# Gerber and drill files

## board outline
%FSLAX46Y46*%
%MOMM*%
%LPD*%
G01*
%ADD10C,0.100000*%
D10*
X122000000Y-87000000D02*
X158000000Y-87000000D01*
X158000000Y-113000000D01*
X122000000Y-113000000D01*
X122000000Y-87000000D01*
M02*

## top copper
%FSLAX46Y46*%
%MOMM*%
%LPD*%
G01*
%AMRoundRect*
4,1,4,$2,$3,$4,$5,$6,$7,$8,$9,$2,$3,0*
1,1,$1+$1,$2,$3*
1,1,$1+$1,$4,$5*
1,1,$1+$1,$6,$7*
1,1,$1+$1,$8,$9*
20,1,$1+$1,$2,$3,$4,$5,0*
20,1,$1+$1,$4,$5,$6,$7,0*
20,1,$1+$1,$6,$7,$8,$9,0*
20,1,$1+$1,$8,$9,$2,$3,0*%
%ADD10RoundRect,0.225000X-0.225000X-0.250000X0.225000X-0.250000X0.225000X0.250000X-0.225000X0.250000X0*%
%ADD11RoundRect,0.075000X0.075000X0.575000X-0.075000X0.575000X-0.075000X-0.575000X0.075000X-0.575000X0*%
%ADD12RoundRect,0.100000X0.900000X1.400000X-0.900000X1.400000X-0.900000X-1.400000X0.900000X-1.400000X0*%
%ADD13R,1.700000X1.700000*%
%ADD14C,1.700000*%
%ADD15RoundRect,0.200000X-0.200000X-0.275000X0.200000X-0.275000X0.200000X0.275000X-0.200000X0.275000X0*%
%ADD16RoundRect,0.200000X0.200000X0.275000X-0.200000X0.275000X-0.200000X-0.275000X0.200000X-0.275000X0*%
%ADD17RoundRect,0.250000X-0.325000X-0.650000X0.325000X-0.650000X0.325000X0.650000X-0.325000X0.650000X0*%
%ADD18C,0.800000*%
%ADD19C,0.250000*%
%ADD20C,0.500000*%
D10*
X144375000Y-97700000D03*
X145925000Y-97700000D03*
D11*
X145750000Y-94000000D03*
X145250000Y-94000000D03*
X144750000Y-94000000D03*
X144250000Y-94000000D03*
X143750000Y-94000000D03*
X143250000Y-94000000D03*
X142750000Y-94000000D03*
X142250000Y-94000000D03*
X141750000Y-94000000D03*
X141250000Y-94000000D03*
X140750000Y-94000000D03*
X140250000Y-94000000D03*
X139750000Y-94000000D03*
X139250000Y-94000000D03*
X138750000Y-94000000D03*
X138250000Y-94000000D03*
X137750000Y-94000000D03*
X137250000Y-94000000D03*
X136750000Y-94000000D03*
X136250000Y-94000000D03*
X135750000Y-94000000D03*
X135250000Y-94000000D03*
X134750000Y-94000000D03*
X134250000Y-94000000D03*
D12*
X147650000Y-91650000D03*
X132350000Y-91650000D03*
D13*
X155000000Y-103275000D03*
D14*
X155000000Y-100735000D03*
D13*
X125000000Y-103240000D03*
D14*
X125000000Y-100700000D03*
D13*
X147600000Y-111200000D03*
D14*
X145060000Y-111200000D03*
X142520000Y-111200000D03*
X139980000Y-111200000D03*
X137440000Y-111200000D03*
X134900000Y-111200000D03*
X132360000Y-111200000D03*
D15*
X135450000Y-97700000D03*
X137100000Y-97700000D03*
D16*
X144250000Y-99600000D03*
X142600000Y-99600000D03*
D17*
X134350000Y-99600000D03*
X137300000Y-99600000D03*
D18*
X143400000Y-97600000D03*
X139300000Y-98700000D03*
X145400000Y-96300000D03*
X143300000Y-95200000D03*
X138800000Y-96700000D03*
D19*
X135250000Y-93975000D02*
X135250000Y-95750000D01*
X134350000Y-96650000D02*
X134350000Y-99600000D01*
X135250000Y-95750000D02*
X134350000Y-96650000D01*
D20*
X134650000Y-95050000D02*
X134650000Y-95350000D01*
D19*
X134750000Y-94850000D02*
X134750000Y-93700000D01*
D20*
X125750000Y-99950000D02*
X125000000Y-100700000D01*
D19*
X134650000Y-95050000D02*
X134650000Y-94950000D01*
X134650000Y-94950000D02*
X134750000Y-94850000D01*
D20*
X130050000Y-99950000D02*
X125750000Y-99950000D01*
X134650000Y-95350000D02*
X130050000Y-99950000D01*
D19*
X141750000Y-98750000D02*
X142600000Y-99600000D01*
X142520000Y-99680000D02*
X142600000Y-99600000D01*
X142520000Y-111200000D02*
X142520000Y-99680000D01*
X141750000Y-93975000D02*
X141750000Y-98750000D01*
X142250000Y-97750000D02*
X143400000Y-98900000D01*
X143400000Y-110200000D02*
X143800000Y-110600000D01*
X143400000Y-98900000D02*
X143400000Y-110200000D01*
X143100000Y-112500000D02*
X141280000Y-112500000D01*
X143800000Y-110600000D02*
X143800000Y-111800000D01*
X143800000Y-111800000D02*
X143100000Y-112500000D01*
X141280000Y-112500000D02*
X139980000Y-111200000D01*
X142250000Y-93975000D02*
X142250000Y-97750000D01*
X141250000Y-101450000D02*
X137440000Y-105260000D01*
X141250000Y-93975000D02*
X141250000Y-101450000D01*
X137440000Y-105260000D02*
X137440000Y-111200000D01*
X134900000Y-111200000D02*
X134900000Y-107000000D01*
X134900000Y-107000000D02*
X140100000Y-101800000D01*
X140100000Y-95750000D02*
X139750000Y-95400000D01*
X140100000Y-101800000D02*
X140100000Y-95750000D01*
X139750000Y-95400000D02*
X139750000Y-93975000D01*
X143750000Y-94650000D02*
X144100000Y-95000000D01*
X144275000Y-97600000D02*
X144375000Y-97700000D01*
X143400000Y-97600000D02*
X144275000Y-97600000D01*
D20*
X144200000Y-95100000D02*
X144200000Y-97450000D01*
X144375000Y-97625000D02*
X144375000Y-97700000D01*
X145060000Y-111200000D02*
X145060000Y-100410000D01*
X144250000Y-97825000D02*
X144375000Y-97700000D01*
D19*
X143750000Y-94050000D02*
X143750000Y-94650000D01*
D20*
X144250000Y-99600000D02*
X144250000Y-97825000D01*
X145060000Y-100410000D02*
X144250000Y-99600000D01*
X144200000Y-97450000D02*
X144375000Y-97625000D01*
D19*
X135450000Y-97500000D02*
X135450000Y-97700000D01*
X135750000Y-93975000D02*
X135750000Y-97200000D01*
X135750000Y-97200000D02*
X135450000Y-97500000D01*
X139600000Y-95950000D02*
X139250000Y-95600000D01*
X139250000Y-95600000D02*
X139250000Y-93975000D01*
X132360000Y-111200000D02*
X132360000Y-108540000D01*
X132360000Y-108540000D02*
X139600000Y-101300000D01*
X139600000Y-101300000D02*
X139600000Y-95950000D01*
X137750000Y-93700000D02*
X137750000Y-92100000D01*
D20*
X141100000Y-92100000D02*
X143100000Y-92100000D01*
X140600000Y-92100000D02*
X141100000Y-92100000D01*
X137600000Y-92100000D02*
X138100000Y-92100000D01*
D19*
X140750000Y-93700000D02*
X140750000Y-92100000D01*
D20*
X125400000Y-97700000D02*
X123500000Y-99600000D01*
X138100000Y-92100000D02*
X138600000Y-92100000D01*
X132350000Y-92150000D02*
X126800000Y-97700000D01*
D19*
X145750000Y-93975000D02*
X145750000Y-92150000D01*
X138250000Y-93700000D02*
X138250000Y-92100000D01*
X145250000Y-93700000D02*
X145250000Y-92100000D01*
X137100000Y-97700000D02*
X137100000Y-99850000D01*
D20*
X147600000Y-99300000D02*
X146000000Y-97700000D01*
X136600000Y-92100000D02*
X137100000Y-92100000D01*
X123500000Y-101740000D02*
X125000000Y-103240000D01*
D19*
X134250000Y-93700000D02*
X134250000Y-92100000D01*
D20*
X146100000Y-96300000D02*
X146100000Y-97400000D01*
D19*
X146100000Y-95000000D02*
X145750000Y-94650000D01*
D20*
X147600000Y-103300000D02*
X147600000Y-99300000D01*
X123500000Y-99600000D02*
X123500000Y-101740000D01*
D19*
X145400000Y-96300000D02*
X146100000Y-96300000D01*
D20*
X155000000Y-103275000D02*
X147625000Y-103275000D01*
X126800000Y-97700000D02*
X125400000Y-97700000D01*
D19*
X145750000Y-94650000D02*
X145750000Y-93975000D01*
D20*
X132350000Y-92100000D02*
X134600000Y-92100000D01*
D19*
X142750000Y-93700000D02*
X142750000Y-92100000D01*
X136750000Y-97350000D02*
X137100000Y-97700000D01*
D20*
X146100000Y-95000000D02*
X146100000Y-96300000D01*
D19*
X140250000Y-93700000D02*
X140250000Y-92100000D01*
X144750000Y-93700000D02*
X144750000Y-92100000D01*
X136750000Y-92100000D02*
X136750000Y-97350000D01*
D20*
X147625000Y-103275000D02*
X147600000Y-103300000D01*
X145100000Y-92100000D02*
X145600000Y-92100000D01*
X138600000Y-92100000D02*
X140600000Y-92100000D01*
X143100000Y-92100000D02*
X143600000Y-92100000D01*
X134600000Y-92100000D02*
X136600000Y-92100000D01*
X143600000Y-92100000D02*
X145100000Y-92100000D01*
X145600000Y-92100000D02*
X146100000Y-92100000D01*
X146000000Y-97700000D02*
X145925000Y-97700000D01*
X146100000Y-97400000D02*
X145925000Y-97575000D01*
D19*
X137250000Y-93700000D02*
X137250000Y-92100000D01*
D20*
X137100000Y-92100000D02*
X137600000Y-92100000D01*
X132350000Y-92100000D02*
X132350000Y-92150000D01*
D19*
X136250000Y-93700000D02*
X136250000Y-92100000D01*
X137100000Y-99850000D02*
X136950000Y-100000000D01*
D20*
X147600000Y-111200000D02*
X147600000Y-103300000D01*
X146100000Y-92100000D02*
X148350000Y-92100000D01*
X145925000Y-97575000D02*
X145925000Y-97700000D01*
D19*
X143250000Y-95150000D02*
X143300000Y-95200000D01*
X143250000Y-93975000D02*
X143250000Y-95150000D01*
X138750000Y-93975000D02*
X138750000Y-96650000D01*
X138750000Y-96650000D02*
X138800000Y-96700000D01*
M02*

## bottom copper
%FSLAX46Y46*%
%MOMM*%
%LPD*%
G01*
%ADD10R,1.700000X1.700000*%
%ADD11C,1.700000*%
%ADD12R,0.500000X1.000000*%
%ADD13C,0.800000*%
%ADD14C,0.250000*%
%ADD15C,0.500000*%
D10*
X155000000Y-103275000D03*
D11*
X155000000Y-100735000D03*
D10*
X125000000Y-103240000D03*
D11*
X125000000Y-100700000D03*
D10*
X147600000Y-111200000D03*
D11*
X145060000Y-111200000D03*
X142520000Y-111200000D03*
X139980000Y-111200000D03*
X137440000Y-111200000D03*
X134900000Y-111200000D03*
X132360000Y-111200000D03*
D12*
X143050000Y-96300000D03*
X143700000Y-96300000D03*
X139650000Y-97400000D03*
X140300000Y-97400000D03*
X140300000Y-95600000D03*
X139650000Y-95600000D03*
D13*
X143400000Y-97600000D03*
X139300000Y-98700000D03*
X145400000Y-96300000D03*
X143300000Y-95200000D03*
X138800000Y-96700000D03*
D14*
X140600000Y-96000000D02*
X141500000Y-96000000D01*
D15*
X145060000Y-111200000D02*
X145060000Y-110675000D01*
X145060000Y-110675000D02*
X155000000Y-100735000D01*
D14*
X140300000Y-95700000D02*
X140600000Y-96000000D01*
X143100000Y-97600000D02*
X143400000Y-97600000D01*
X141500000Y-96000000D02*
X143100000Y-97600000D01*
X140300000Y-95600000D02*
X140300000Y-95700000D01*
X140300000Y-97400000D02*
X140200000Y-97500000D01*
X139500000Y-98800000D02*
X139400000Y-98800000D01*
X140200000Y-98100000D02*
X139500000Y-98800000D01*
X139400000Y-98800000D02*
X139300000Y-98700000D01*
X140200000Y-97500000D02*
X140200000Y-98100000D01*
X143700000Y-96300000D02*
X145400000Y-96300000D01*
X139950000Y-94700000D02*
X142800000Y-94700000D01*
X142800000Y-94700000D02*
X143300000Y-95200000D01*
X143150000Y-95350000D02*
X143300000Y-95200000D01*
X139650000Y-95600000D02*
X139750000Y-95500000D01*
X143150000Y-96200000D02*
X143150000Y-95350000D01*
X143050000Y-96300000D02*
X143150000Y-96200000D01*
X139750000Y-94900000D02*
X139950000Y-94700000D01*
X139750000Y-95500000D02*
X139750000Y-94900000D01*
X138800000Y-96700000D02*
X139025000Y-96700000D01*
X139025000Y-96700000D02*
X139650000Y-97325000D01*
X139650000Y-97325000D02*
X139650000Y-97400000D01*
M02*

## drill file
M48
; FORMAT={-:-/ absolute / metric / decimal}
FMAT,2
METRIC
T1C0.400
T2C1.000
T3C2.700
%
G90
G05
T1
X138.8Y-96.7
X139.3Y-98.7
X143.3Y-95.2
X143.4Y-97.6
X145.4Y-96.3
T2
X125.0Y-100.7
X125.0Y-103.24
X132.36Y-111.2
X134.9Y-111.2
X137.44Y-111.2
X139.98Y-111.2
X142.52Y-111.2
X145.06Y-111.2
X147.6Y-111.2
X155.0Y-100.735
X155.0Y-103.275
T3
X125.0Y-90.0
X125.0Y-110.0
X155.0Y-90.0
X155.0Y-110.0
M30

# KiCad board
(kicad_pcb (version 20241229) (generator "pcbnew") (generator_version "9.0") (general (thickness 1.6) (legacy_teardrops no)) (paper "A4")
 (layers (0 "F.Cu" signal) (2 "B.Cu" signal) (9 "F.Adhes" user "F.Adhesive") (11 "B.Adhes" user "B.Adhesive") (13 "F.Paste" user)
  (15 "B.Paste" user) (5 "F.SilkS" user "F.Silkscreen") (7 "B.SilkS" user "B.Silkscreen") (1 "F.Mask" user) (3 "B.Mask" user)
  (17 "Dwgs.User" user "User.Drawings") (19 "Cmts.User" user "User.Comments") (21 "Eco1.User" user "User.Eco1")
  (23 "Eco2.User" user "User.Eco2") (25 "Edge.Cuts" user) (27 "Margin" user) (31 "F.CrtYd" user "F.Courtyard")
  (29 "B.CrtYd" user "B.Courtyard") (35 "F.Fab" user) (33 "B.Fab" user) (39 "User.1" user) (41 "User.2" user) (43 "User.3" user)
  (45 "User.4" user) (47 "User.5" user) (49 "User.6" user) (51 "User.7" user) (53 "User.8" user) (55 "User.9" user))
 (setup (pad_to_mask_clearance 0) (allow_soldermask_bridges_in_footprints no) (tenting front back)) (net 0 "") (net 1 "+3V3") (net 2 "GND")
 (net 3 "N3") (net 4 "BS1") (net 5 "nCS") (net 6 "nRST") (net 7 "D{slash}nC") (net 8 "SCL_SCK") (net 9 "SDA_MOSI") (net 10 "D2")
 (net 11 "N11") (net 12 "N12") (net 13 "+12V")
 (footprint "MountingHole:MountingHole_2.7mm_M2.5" (layer "F.Cu") (at 155 110)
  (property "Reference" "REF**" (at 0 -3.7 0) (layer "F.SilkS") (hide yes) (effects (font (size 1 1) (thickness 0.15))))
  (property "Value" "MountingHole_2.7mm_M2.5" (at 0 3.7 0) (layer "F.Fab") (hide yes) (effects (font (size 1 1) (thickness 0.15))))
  (pad "" np_thru_hole circle (at 0 0) (size 2.7 2.7) (drill 2.7) (layers "*.Cu" "*.Mask")))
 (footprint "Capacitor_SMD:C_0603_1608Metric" (layer "F.Cu") (at 145.15 97.7)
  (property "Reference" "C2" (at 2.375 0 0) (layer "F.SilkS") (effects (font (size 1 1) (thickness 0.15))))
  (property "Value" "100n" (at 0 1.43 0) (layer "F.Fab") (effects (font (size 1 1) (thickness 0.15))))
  (pad "1" smd roundrect (at -0.775 0) (size 0.9 0.95) (layers "F.Cu" "F.Mask" "F.Paste") (roundrect_rratio 0.25) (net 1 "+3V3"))
  (pad "2" smd roundrect (at 0.775 0) (size 0.9 0.95) (layers "F.Cu" "F.Mask" "F.Paste") (roundrect_rratio 0.25) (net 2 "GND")))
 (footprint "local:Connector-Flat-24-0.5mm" (layer "F.Cu") (at 140 92.9 180)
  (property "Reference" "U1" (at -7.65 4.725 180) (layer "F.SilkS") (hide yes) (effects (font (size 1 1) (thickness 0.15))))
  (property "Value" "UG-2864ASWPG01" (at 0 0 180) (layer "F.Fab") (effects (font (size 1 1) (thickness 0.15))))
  (pad "1" smd roundrect (at -5.75 -1.1 180) (size 0.3 1.3) (layers "F.Cu" "F.Mask" "F.Paste") (roundrect_rratio 0.25) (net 2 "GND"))
  (pad "2" smd roundrect (at -5.25 -1.1 180) (size 0.3 1.3) (layers "F.Cu" "F.Mask" "F.Paste") (roundrect_rratio 0.25) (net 2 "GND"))
  (pad "3" smd roundrect (at -4.75 -1.1 180) (size 0.3 1.3) (layers "F.Cu" "F.Mask" "F.Paste") (roundrect_rratio 0.25) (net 2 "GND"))
  (pad "4" smd roundrect (at -4.25 -1.1 180) (size 0.3 1.3) (layers "F.Cu" "F.Mask" "F.Paste") (roundrect_rratio 0.25) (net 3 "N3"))
  (pad "5" smd roundrect (at -3.75 -1.1 180) (size 0.3 1.3) (layers "F.Cu" "F.Mask" "F.Paste") (roundrect_rratio 0.25) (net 1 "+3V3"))
  (pad "6" smd roundrect (at -3.25 -1.1 180) (size 0.3 1.3) (layers "F.Cu" "F.Mask" "F.Paste") (roundrect_rratio 0.25) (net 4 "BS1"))
  (pad "7" smd roundrect (at -2.75 -1.1 180) (size 0.3 1.3) (layers "F.Cu" "F.Mask" "F.Paste") (roundrect_rratio 0.25) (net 2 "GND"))
  (pad "8" smd roundrect (at -2.25 -1.1 180) (size 0.3 1.3) (layers "F.Cu" "F.Mask" "F.Paste") (roundrect_rratio 0.25) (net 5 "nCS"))
  (pad "9" smd roundrect (at -1.75 -1.1 180) (size 0.3 1.3) (layers "F.Cu" "F.Mask" "F.Paste") (roundrect_rratio 0.25) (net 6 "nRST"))
  (pad "10" smd roundrect (at -1.25 -1.1 180) (size 0.3 1.3) (layers "F.Cu" "F.Mask" "F.Paste") (roundrect_rratio 0.25) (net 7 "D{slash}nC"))
  (pad "11" smd roundrect (at -0.75 -1.1 180) (size 0.3 1.3) (layers "F.Cu" "F.Mask" "F.Paste") (roundrect_rratio 0.25) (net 2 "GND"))
  (pad "12" smd roundrect (at -0.25 -1.1 180) (size 0.3 1.3) (layers "F.Cu" "F.Mask" "F.Paste") (roundrect_rratio 0.25) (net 2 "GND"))
  (pad "13" smd roundrect (at 0.25 -1.1 180) (size 0.3 1.3) (layers "F.Cu" "F.Mask" "F.Paste") (roundrect_rratio 0.25) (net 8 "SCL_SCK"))
  (pad "14" smd roundrect (at 0.75 -1.1 180) (size 0.3 1.3) (layers "F.Cu" "F.Mask" "F.Paste") (roundrect_rratio 0.25) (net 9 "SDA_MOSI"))
  (pad "15" smd roundrect (at 1.25 -1.1 180) (size 0.3 1.3) (layers "F.Cu" "F.Mask" "F.Paste") (roundrect_rratio 0.25) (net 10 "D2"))
  (pad "16" smd roundrect (at 1.75 -1.1 180) (size 0.3 1.3) (layers "F.Cu" "F.Mask" "F.Paste") (roundrect_rratio 0.25) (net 2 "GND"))
  (pad "17" smd roundrect (at 2.25 -1.1 180) (size 0.3 1.3) (layers "F.Cu" "F.Mask" "F.Paste") (roundrect_rratio 0.25) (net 2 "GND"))
  (pad "18" smd roundrect (at 2.75 -1.1 180) (size 0.3 1.3) (layers "F.Cu" "F.Mask" "F.Paste") (roundrect_rratio 0.25) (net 2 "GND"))
  (pad "19" smd roundrect (at 3.25 -1.1 180) (size 0.3 1.3) (layers "F.Cu" "F.Mask" "F.Paste") (roundrect_rratio 0.25) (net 2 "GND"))
  (pad "20" smd roundrect (at 3.75 -1.1 180) (size 0.3 1.3) (layers "F.Cu" "F.Mask" "F.Paste") (roundrect_rratio 0.25) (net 2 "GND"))
  (pad "21" smd roundrect (at 4.25 -1.1 180) (size 0.3 1.3) (layers "F.Cu" "F.Mask" "F.Paste") (roundrect_rratio 0.25) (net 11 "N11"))
  (pad "22" smd roundrect (at 4.75 -1.1 180) (size 0.3 1.3) (layers "F.Cu" "F.Mask" "F.Paste") (roundrect_rratio 0.25) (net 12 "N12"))
  (pad "23" smd roundrect (at 5.25 -1.1 180) (size 0.3 1.3) (layers "F.Cu" "F.Mask" "F.Paste") (roundrect_rratio 0.25) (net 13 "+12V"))
  (pad "24" smd roundrect (at 5.75 -1.1 180) (size 0.3 1.3) (layers "F.Cu" "F.Mask" "F.Paste") (roundrect_rratio 0.25) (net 2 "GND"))
  (pad "25" smd roundrect (at -7.65 1.25 180) (size 2 3) (layers "F.Cu" "F.Mask" "F.Paste") (roundrect_rratio 0.05) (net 2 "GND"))
  (pad "26" smd roundrect (at 7.65 1.25 180) (size 2 3) (layers "F.Cu" "F.Mask" "F.Paste") (roundrect_rratio 0.05) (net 2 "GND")))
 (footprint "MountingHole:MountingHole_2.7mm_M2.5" (layer "F.Cu") (at 125 110)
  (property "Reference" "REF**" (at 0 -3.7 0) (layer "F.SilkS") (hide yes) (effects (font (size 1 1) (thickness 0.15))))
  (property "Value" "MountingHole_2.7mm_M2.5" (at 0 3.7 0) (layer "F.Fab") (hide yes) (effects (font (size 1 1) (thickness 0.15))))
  (pad "" np_thru_hole circle (at 0 0) (size 2.7 2.7) (drill 2.7) (layers "*.Cu" "*.Mask")))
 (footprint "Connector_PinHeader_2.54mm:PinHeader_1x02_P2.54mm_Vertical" (layer "F.Cu") (at 155 103.275 180)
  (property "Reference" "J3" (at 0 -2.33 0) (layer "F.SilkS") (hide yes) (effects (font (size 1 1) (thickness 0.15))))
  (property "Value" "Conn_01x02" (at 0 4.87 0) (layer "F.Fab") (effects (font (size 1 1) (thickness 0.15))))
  (pad "1" thru_hole rect (at 0 0 180) (size 1.7 1.7) (drill 1) (layers "*.Cu" "*.Mask") (remove_unused_layers no) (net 2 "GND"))
  (pad "2" thru_hole circle (at 0 2.54 180) (size 1.7 1.7) (drill 1) (layers "*.Cu" "*.Mask") (remove_unused_layers no) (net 1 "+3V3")))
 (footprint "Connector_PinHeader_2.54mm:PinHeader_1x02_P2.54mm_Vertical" (layer "F.Cu") (at 125 103.24 180)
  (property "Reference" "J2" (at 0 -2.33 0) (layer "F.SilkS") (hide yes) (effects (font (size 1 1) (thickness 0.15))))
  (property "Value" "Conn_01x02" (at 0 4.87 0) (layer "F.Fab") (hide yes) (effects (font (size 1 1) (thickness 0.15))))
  (pad "1" thru_hole rect (at 0 0 180) (size 1.7 1.7) (drill 1) (layers "*.Cu" "*.Mask") (remove_unused_layers no) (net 2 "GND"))
  (pad "2" thru_hole circle (at 0 2.54 180) (size 1.7 1.7) (drill 1) (layers "*.Cu" "*.Mask") (remove_unused_layers no) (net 13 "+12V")))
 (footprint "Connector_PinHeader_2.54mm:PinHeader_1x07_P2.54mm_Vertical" (layer "F.Cu") (at 147.6 111.2 -90)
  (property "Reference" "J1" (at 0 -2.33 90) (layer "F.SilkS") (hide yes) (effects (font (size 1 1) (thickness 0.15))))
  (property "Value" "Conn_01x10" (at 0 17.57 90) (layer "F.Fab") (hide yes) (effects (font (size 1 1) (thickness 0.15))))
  (pad "1" thru_hole rect (at 0 0 270) (size 1.7 1.7) (drill 1) (layers "*.Cu" "*.Mask") (remove_unused_layers no) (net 2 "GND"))
  (pad "2" thru_hole circle (at 0 2.54 270) (size 1.7 1.7) (drill 1) (layers "*.Cu" "*.Mask") (remove_unused_layers no) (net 1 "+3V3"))
  (pad "3" thru_hole circle (at 0 5.08 270) (size 1.7 1.7) (drill 1) (layers "*.Cu" "*.Mask") (remove_unused_layers no) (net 6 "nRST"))
  (pad "4" thru_hole circle (at 0 7.62 270) (size 1.7 1.7) (drill 1) (layers "*.Cu" "*.Mask") (remove_unused_layers no) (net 5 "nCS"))
  (pad "5" thru_hole circle (at 0 10.16 270) (size 1.7 1.7) (drill 1) (layers "*.Cu" "*.Mask") (remove_unused_layers no)
   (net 7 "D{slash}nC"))
  (pad "6" thru_hole circle (at 0 12.7 270) (size 1.7 1.7) (drill 1) (layers "*.Cu" "*.Mask") (remove_unused_layers no) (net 8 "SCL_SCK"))
  (pad "7" thru_hole circle (at 0 15.24 270) (size 1.7 1.7) (drill 1) (layers "*.Cu" "*.Mask") (remove_unused_layers no) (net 9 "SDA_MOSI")))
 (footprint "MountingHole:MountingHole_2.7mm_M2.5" (layer "F.Cu") (at 155 90)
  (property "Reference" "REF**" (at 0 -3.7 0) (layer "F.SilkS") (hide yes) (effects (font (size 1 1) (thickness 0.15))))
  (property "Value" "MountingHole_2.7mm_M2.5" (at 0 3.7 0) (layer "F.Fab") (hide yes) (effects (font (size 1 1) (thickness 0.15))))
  (pad "" np_thru_hole circle (at 0 0) (size 2.7 2.7) (drill 2.7) (layers "*.Cu" "*.Mask")))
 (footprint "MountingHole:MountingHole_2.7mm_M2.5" (layer "F.Cu") (at 125 90)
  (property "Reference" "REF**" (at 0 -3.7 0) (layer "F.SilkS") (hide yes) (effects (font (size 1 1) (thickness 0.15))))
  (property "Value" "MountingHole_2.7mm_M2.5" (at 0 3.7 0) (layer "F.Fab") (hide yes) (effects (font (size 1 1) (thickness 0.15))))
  (pad "" np_thru_hole circle (at 0 0) (size 2.7 2.7) (drill 2.7) (layers "*.Cu" "*.Mask")))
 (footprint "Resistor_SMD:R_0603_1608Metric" (layer "F.Cu") (at 136.275 97.7)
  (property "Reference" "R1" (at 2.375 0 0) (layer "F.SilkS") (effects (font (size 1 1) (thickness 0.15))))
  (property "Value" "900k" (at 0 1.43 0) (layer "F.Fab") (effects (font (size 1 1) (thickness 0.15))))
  (pad "1" smd roundrect (at -0.825 0) (size 0.8 0.95) (layers "F.Cu" "F.Mask" "F.Paste") (roundrect_rratio 0.25) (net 11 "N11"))
  (pad "2" smd roundrect (at 0.825 0) (size 0.8 0.95) (layers "F.Cu" "F.Mask" "F.Paste") (roundrect_rratio 0.25) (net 2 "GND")))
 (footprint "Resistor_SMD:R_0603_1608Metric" (layer "F.Cu") (at 143.425 99.6 180)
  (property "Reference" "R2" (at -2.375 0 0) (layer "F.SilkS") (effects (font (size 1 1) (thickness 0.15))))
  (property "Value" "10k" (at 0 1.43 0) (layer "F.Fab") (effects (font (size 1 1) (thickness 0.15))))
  (pad "1" smd roundrect (at -0.825 0 180) (size 0.8 0.95) (layers "F.Cu" "F.Mask" "F.Paste") (roundrect_rratio 0.25) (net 1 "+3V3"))
  (pad "2" smd roundrect (at 0.825 0 180) (size 0.8 0.95) (layers "F.Cu" "F.Mask" "F.Paste") (roundrect_rratio 0.25) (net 6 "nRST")))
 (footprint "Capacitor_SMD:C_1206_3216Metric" (layer "F.Cu") (at 135.825 99.6)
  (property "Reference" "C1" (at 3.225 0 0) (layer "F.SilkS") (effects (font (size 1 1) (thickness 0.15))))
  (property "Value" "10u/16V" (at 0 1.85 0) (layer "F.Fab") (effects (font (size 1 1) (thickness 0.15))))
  (pad "1" smd roundrect (at -1.475 0) (size 1.15 1.8) (layers "F.Cu" "F.Mask" "F.Paste") (roundrect_rratio 0.217391) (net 12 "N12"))
  (pad "2" smd roundrect (at 1.475 0) (size 1.15 1.8) (layers "F.Cu" "F.Mask" "F.Paste") (roundrect_rratio 0.217391) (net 2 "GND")))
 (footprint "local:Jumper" (layer "B.Cu") (at 143.375 96.3)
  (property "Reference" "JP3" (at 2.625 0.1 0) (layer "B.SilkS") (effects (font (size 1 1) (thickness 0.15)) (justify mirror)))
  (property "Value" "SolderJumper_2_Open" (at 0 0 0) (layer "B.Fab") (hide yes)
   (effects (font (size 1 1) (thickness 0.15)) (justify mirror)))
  (pad "1" smd rect (at -0.325 0) (size 0.5 1) (layers "B.Cu") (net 4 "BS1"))
  (pad "2" smd rect (at 0.325 0) (size 0.5 1) (layers "B.Cu") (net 2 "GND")))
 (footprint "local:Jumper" (layer "B.Cu") (at 139.975 97.4)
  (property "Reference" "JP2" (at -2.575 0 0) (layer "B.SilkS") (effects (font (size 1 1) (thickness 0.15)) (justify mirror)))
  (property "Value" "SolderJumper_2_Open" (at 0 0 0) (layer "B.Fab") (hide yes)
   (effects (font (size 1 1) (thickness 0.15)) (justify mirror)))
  (pad "1" smd rect (at -0.325 0) (size 0.5 1) (layers "B.Cu") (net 10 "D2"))
  (pad "2" smd rect (at 0.325 0) (size 0.5 1) (layers "B.Cu") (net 9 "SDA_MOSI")))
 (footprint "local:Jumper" (layer "B.Cu") (at 139.975 95.6 180)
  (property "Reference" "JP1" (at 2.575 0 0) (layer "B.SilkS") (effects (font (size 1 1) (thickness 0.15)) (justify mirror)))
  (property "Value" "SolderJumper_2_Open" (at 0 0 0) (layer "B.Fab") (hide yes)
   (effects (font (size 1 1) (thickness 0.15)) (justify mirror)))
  (pad "1" smd rect (at -0.325 0 180) (size 0.5 1) (layers "B.Cu") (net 1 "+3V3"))
  (pad "2" smd rect (at 0.325 0 180) (size 0.5 1) (layers "B.Cu") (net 4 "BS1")))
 (gr_rect (start 122 87) (end 158 113) (stroke (width 0.1) (type default)) (fill no) (layer "Edge.Cuts"))
 (segment (start 135.25 93.975) (end 135.25 95.75) (width 0.25) (layer "F.Cu") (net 12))
 (segment (start 134.35 96.65) (end 134.35 99.6) (width 0.25) (layer "F.Cu") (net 12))
 (segment (start 135.25 95.75) (end 134.35 96.65) (width 0.25) (layer "F.Cu") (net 12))
 (segment (start 134.65 95.05) (end 134.65 95.35) (width 0.5) (layer "F.Cu") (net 13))
 (segment (start 134.75 94.85) (end 134.75 93.7) (width 0.25) (layer "F.Cu") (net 13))
 (segment (start 125.75 99.95) (end 125 100.7) (width 0.5) (layer "F.Cu") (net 13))
 (segment (start 134.65 95.05) (end 134.65 94.95) (width 0.25) (layer "F.Cu") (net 13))
 (segment (start 134.65 94.95) (end 134.75 94.85) (width 0.25) (layer "F.Cu") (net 13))
 (segment (start 130.05 99.95) (end 125.75 99.95) (width 0.5) (layer "F.Cu") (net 13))
 (segment (start 134.65 95.35) (end 130.05 99.95) (width 0.5) (layer "F.Cu") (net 13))
 (segment (start 141.75 98.75) (end 142.6 99.6) (width 0.25) (layer "F.Cu") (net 6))
 (segment (start 142.52 99.68) (end 142.6 99.6) (width 0.25) (layer "F.Cu") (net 6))
 (segment (start 142.52 111.2) (end 142.52 99.68) (width 0.25) (layer "F.Cu") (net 6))
 (segment (start 141.75 93.975) (end 141.75 98.75) (width 0.25) (layer "F.Cu") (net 6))
 (segment (start 142.25 97.75) (end 143.4 98.9) (width 0.25) (layer "F.Cu") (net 5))
 (segment (start 143.4 110.2) (end 143.8 110.6) (width 0.25) (layer "F.Cu") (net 5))
 (segment (start 143.4 98.9) (end 143.4 110.2) (width 0.25) (layer "F.Cu") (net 5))
 (segment (start 143.1 112.5) (end 141.28 112.5) (width 0.25) (layer "F.Cu") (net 5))
 (segment (start 143.8 110.6) (end 143.8 111.8) (width 0.25) (layer "F.Cu") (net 5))
 (segment (start 143.8 111.8) (end 143.1 112.5) (width 0.25) (layer "F.Cu") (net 5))
 (segment (start 141.28 112.5) (end 139.98 111.2) (width 0.25) (layer "F.Cu") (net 5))
 (segment (start 142.25 93.975) (end 142.25 97.75) (width 0.25) (layer "F.Cu") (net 5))
 (segment (start 141.25 101.45) (end 137.44 105.26) (width 0.25) (layer "F.Cu") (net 7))
 (segment (start 141.25 93.975) (end 141.25 101.45) (width 0.25) (layer "F.Cu") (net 7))
 (segment (start 137.44 105.26) (end 137.44 111.2) (width 0.25) (layer "F.Cu") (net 7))
 (segment (start 134.9 111.2) (end 134.9 107) (width 0.25) (layer "F.Cu") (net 8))
 (segment (start 134.9 107) (end 140.1 101.8) (width 0.25) (layer "F.Cu") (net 8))
 (segment (start 140.1 95.75) (end 139.75 95.4) (width 0.25) (layer "F.Cu") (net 8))
 (segment (start 140.1 101.8) (end 140.1 95.75) (width 0.25) (layer "F.Cu") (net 8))
 (segment (start 139.75 95.4) (end 139.75 93.975) (width 0.25) (layer "F.Cu") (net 8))
 (segment (start 143.75 94.65) (end 144.1 95) (width 0.25) (layer "F.Cu") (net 1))
 (segment (start 144.275 97.6) (end 144.375 97.7) (width 0.25) (layer "F.Cu") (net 1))
 (segment (start 143.4 97.6) (end 144.275 97.6) (width 0.25) (layer "F.Cu") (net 1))
 (segment (start 144.2 95.1) (end 144.2 97.45) (width 0.5) (layer "F.Cu") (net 1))
 (segment (start 144.375 97.625) (end 144.375 97.7) (width 0.5) (layer "F.Cu") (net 1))
 (segment (start 145.06 111.2) (end 145.06 100.41) (width 0.5) (layer "F.Cu") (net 1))
 (segment (start 144.25 97.825) (end 144.375 97.7) (width 0.5) (layer "F.Cu") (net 1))
 (segment (start 143.75 94.05) (end 143.75 94.65) (width 0.25) (layer "F.Cu") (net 1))
 (segment (start 144.25 99.6) (end 144.25 97.825) (width 0.5) (layer "F.Cu") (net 1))
 (segment (start 145.06 100.41) (end 144.25 99.6) (width 0.5) (layer "F.Cu") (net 1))
 (segment (start 144.2 97.45) (end 144.375 97.625) (width 0.5) (layer "F.Cu") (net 1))
 (via (at 143.4 97.6) (size 0.8) (drill 0.4) (layers "F.Cu" "B.Cu") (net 1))
 (segment (start 140.6 96) (end 141.5 96) (width 0.25) (layer "B.Cu") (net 1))
 (segment (start 145.06 111.2) (end 145.06 110.675) (width 0.5) (layer "B.Cu") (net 1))
 (segment (start 145.06 110.675) (end 155 100.735) (width 0.5) (layer "B.Cu") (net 1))
 (segment (start 140.3 95.7) (end 140.6 96) (width 0.25) (layer "B.Cu") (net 1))
 (segment (start 143.1 97.6) (end 143.4 97.6) (width 0.25) (layer "B.Cu") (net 1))
 (segment (start 141.5 96) (end 143.1 97.6) (width 0.25) (layer "B.Cu") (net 1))
 (segment (start 140.3 95.6) (end 140.3 95.7) (width 0.25) (layer "B.Cu") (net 1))
 (segment (start 135.45 97.5) (end 135.45 97.7) (width 0.25) (layer "F.Cu") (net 11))
 (segment (start 135.75 93.975) (end 135.75 97.2) (width 0.25) (layer "F.Cu") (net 11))
 (segment (start 135.75 97.2) (end 135.45 97.5) (width 0.25) (layer "F.Cu") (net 11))
 (segment (start 139.6 95.95) (end 139.25 95.6) (width 0.25) (layer "F.Cu") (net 9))
 (segment (start 139.25 95.6) (end 139.25 93.975) (width 0.25) (layer "F.Cu") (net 9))
 (segment (start 132.36 111.2) (end 132.36 108.54) (width 0.25) (layer "F.Cu") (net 9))
 (segment (start 132.36 108.54) (end 139.6 101.3) (width 0.25) (layer "F.Cu") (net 9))
 (segment (start 139.6 101.3) (end 139.6 95.95) (width 0.25) (layer "F.Cu") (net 9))
 (via (at 139.3 98.7) (size 0.8) (drill 0.4) (layers "F.Cu" "B.Cu") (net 9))
 (segment (start 140.3 97.4) (end 140.2 97.5) (width 0.25) (layer "B.Cu") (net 9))
 (segment (start 139.5 98.8) (end 139.4 98.8) (width 0.25) (layer "B.Cu") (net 9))
 (segment (start 140.2 98.1) (end 139.5 98.8) (width 0.25) (layer "B.Cu") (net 9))
 (segment (start 139.4 98.8) (end 139.3 98.7) (width 0.25) (layer "B.Cu") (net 9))
 (segment (start 140.2 97.5) (end 140.2 98.1) (width 0.25) (layer "B.Cu") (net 9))
 (segment (start 137.75 93.7) (end 137.75 92.1) (width 0.25) (layer "F.Cu") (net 2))
 (segment (start 141.1 92.1) (end 143.1 92.1) (width 0.5) (layer "F.Cu") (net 2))
 (segment (start 140.6 92.1) (end 141.1 92.1) (width 0.5) (layer "F.Cu") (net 2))
 (segment (start 137.6 92.1) (end 138.1 92.1) (width 0.5) (layer "F.Cu") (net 2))
 (segment (start 140.75 93.7) (end 140.75 92.1) (width 0.25) (layer "F.Cu") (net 2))
 (segment (start 125.4 97.7) (end 123.5 99.6) (width 0.5) (layer "F.Cu") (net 2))
 (segment (start 138.1 92.1) (end 138.6 92.1) (width 0.5) (layer "F.Cu") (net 2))
 (segment (start 132.35 92.15) (end 126.8 97.7) (width 0.5) (layer "F.Cu") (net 2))
 (segment (start 145.75 93.975) (end 145.75 92.15) (width 0.25) (layer "F.Cu") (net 2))
 (segment (start 138.25 93.7) (end 138.25 92.1) (width 0.25) (layer "F.Cu") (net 2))
 (segment (start 145.25 93.7) (end 145.25 92.1) (width 0.25) (layer "F.Cu") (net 2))
 (segment (start 137.1 97.7) (end 137.1 99.85) (width 0.25) (layer "F.Cu") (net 2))
 (segment (start 147.6 99.3) (end 146 97.7) (width 0.5) (layer "F.Cu") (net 2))
 (segment (start 136.6 92.1) (end 137.1 92.1) (width 0.5) (layer "F.Cu") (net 2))
 (segment (start 123.5 101.74) (end 125 103.24) (width 0.5) (layer "F.Cu") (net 2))
 (segment (start 134.25 93.7) (end 134.25 92.1) (width 0.25) (layer "F.Cu") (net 2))
 (segment (start 146.1 96.3) (end 146.1 97.4) (width 0.5) (layer "F.Cu") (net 2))
 (segment (start 146.1 95) (end 145.75 94.65) (width 0.25) (layer "F.Cu") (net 2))
 (segment (start 147.6 103.3) (end 147.6 99.3) (width 0.5) (layer "F.Cu") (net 2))
 (segment (start 123.5 99.6) (end 123.5 101.74) (width 0.5) (layer "F.Cu") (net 2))
 (segment (start 145.4 96.3) (end 146.1 96.3) (width 0.25) (layer "F.Cu") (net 2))
 (segment (start 155 103.275) (end 147.625 103.275) (width 0.5) (layer "F.Cu") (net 2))
 (segment (start 126.8 97.7) (end 125.4 97.7) (width 0.5) (layer "F.Cu") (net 2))
 (segment (start 145.75 94.65) (end 145.75 93.975) (width 0.25) (layer "F.Cu") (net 2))
 (segment (start 132.35 92.1) (end 134.6 92.1) (width 0.5) (layer "F.Cu") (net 2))
 (segment (start 142.75 93.7) (end 142.75 92.1) (width 0.25) (layer "F.Cu") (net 2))
 (segment (start 136.75 97.35) (end 137.1 97.7) (width 0.25) (layer "F.Cu") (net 2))
 (segment (start 146.1 95) (end 146.1 96.3) (width 0.5) (layer "F.Cu") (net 2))
 (segment (start 140.25 93.7) (end 140.25 92.1) (width 0.25) (layer "F.Cu") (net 2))
 (segment (start 144.75 93.7) (end 144.75 92.1) (width 0.25) (layer "F.Cu") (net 2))
 (segment (start 136.75 92.1) (end 136.75 97.35) (width 0.25) (layer "F.Cu") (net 2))
 (segment (start 147.625 103.275) (end 147.6 103.3) (width 0.5) (layer "F.Cu") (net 2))
 (segment (start 145.1 92.1) (end 145.6 92.1) (width 0.5) (layer "F.Cu") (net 2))
 (segment (start 138.6 92.1) (end 140.6 92.1) (width 0.5) (layer "F.Cu") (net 2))
 (segment (start 143.1 92.1) (end 143.6 92.1) (width 0.5) (layer "F.Cu") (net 2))
 (segment (start 134.6 92.1) (end 136.6 92.1) (width 0.5) (layer "F.Cu") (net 2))
 (segment (start 143.6 92.1) (end 145.1 92.1) (width 0.5) (layer "F.Cu") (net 2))
 (segment (start 145.6 92.1) (end 146.1 92.1) (width 0.5) (layer "F.Cu") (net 2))
 (segment (start 146 97.7) (end 145.925 97.7) (width 0.5) (layer "F.Cu") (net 2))
 (segment (start 146.1 97.4) (end 145.925 97.575) (width 0.5) (layer "F.Cu") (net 2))
 (segment (start 137.25 93.7) (end 137.25 92.1) (width 0.25) (layer "F.Cu") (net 2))
 (segment (start 137.1 92.1) (end 137.6 92.1) (width 0.5) (layer "F.Cu") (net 2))
 (segment (start 132.35 92.1) (end 132.35 92.15) (width 0.5) (layer "F.Cu") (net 2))
 (segment (start 136.25 93.7) (end 136.25 92.1) (width 0.25) (layer "F.Cu") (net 2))
 (segment (start 137.1 99.85) (end 136.95 100) (width 0.25) (layer "F.Cu") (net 2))
 (segment (start 147.6 111.2) (end 147.6 103.3) (width 0.5) (layer "F.Cu") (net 2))
 (segment (start 146.1 92.1) (end 148.35 92.1) (width 0.5) (layer "F.Cu") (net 2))
 (segment (start 145.925 97.575) (end 145.925 97.7) (width 0.5) (layer "F.Cu") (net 2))
 (via (at 145.4 96.3) (size 0.8) (drill 0.4) (layers "F.Cu" "B.Cu") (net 2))
 (segment (start 143.7 96.3) (end 145.4 96.3) (width 0.25) (layer "B.Cu") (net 2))
 (segment (start 143.25 95.15) (end 143.3 95.2) (width 0.25) (layer "F.Cu") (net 4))
 (segment (start 143.25 93.975) (end 143.25 95.15) (width 0.25) (layer "F.Cu") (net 4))
 (via (at 143.3 95.2) (size 0.8) (drill 0.4) (layers "F.Cu" "B.Cu") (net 4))
 (segment (start 139.95 94.7) (end 142.8 94.7) (width 0.25) (layer "B.Cu") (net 4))
 (segment (start 142.8 94.7) (end 143.3 95.2) (width 0.25) (layer "B.Cu") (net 4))
 (segment (start 143.15 95.35) (end 143.3 95.2) (width 0.25) (layer "B.Cu") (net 4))
 (segment (start 139.65 95.6) (end 139.75 95.5) (width 0.25) (layer "B.Cu") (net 4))
 (segment (start 143.15 96.2) (end 143.15 95.35) (width 0.25) (layer "B.Cu") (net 4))
 (segment (start 143.05 96.3) (end 143.15 96.2) (width 0.25) (layer "B.Cu") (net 4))
 (segment (start 139.75 94.9) (end 139.95 94.7) (width 0.25) (layer "B.Cu") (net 4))
 (segment (start 139.75 95.5) (end 139.75 94.9) (width 0.25) (layer "B.Cu") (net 4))
 (segment (start 138.75 93.975) (end 138.75 96.65) (width 0.25) (layer "F.Cu") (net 10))
 (segment (start 138.75 96.65) (end 138.8 96.7) (width 0.25) (layer "F.Cu") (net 10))
 (via (at 138.8 96.7) (size 0.8) (drill 0.4) (layers "F.Cu" "B.Cu") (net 10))
 (segment (start 138.8 96.7) (end 139.025 96.7) (width 0.25) (layer "B.Cu") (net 10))
 (segment (start 139.025 96.7) (end 139.65 97.325) (width 0.25) (layer "B.Cu") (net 10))
 (segment (start 139.65 97.325) (end 139.65 97.4) (width 0.25) (layer "B.Cu") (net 10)))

